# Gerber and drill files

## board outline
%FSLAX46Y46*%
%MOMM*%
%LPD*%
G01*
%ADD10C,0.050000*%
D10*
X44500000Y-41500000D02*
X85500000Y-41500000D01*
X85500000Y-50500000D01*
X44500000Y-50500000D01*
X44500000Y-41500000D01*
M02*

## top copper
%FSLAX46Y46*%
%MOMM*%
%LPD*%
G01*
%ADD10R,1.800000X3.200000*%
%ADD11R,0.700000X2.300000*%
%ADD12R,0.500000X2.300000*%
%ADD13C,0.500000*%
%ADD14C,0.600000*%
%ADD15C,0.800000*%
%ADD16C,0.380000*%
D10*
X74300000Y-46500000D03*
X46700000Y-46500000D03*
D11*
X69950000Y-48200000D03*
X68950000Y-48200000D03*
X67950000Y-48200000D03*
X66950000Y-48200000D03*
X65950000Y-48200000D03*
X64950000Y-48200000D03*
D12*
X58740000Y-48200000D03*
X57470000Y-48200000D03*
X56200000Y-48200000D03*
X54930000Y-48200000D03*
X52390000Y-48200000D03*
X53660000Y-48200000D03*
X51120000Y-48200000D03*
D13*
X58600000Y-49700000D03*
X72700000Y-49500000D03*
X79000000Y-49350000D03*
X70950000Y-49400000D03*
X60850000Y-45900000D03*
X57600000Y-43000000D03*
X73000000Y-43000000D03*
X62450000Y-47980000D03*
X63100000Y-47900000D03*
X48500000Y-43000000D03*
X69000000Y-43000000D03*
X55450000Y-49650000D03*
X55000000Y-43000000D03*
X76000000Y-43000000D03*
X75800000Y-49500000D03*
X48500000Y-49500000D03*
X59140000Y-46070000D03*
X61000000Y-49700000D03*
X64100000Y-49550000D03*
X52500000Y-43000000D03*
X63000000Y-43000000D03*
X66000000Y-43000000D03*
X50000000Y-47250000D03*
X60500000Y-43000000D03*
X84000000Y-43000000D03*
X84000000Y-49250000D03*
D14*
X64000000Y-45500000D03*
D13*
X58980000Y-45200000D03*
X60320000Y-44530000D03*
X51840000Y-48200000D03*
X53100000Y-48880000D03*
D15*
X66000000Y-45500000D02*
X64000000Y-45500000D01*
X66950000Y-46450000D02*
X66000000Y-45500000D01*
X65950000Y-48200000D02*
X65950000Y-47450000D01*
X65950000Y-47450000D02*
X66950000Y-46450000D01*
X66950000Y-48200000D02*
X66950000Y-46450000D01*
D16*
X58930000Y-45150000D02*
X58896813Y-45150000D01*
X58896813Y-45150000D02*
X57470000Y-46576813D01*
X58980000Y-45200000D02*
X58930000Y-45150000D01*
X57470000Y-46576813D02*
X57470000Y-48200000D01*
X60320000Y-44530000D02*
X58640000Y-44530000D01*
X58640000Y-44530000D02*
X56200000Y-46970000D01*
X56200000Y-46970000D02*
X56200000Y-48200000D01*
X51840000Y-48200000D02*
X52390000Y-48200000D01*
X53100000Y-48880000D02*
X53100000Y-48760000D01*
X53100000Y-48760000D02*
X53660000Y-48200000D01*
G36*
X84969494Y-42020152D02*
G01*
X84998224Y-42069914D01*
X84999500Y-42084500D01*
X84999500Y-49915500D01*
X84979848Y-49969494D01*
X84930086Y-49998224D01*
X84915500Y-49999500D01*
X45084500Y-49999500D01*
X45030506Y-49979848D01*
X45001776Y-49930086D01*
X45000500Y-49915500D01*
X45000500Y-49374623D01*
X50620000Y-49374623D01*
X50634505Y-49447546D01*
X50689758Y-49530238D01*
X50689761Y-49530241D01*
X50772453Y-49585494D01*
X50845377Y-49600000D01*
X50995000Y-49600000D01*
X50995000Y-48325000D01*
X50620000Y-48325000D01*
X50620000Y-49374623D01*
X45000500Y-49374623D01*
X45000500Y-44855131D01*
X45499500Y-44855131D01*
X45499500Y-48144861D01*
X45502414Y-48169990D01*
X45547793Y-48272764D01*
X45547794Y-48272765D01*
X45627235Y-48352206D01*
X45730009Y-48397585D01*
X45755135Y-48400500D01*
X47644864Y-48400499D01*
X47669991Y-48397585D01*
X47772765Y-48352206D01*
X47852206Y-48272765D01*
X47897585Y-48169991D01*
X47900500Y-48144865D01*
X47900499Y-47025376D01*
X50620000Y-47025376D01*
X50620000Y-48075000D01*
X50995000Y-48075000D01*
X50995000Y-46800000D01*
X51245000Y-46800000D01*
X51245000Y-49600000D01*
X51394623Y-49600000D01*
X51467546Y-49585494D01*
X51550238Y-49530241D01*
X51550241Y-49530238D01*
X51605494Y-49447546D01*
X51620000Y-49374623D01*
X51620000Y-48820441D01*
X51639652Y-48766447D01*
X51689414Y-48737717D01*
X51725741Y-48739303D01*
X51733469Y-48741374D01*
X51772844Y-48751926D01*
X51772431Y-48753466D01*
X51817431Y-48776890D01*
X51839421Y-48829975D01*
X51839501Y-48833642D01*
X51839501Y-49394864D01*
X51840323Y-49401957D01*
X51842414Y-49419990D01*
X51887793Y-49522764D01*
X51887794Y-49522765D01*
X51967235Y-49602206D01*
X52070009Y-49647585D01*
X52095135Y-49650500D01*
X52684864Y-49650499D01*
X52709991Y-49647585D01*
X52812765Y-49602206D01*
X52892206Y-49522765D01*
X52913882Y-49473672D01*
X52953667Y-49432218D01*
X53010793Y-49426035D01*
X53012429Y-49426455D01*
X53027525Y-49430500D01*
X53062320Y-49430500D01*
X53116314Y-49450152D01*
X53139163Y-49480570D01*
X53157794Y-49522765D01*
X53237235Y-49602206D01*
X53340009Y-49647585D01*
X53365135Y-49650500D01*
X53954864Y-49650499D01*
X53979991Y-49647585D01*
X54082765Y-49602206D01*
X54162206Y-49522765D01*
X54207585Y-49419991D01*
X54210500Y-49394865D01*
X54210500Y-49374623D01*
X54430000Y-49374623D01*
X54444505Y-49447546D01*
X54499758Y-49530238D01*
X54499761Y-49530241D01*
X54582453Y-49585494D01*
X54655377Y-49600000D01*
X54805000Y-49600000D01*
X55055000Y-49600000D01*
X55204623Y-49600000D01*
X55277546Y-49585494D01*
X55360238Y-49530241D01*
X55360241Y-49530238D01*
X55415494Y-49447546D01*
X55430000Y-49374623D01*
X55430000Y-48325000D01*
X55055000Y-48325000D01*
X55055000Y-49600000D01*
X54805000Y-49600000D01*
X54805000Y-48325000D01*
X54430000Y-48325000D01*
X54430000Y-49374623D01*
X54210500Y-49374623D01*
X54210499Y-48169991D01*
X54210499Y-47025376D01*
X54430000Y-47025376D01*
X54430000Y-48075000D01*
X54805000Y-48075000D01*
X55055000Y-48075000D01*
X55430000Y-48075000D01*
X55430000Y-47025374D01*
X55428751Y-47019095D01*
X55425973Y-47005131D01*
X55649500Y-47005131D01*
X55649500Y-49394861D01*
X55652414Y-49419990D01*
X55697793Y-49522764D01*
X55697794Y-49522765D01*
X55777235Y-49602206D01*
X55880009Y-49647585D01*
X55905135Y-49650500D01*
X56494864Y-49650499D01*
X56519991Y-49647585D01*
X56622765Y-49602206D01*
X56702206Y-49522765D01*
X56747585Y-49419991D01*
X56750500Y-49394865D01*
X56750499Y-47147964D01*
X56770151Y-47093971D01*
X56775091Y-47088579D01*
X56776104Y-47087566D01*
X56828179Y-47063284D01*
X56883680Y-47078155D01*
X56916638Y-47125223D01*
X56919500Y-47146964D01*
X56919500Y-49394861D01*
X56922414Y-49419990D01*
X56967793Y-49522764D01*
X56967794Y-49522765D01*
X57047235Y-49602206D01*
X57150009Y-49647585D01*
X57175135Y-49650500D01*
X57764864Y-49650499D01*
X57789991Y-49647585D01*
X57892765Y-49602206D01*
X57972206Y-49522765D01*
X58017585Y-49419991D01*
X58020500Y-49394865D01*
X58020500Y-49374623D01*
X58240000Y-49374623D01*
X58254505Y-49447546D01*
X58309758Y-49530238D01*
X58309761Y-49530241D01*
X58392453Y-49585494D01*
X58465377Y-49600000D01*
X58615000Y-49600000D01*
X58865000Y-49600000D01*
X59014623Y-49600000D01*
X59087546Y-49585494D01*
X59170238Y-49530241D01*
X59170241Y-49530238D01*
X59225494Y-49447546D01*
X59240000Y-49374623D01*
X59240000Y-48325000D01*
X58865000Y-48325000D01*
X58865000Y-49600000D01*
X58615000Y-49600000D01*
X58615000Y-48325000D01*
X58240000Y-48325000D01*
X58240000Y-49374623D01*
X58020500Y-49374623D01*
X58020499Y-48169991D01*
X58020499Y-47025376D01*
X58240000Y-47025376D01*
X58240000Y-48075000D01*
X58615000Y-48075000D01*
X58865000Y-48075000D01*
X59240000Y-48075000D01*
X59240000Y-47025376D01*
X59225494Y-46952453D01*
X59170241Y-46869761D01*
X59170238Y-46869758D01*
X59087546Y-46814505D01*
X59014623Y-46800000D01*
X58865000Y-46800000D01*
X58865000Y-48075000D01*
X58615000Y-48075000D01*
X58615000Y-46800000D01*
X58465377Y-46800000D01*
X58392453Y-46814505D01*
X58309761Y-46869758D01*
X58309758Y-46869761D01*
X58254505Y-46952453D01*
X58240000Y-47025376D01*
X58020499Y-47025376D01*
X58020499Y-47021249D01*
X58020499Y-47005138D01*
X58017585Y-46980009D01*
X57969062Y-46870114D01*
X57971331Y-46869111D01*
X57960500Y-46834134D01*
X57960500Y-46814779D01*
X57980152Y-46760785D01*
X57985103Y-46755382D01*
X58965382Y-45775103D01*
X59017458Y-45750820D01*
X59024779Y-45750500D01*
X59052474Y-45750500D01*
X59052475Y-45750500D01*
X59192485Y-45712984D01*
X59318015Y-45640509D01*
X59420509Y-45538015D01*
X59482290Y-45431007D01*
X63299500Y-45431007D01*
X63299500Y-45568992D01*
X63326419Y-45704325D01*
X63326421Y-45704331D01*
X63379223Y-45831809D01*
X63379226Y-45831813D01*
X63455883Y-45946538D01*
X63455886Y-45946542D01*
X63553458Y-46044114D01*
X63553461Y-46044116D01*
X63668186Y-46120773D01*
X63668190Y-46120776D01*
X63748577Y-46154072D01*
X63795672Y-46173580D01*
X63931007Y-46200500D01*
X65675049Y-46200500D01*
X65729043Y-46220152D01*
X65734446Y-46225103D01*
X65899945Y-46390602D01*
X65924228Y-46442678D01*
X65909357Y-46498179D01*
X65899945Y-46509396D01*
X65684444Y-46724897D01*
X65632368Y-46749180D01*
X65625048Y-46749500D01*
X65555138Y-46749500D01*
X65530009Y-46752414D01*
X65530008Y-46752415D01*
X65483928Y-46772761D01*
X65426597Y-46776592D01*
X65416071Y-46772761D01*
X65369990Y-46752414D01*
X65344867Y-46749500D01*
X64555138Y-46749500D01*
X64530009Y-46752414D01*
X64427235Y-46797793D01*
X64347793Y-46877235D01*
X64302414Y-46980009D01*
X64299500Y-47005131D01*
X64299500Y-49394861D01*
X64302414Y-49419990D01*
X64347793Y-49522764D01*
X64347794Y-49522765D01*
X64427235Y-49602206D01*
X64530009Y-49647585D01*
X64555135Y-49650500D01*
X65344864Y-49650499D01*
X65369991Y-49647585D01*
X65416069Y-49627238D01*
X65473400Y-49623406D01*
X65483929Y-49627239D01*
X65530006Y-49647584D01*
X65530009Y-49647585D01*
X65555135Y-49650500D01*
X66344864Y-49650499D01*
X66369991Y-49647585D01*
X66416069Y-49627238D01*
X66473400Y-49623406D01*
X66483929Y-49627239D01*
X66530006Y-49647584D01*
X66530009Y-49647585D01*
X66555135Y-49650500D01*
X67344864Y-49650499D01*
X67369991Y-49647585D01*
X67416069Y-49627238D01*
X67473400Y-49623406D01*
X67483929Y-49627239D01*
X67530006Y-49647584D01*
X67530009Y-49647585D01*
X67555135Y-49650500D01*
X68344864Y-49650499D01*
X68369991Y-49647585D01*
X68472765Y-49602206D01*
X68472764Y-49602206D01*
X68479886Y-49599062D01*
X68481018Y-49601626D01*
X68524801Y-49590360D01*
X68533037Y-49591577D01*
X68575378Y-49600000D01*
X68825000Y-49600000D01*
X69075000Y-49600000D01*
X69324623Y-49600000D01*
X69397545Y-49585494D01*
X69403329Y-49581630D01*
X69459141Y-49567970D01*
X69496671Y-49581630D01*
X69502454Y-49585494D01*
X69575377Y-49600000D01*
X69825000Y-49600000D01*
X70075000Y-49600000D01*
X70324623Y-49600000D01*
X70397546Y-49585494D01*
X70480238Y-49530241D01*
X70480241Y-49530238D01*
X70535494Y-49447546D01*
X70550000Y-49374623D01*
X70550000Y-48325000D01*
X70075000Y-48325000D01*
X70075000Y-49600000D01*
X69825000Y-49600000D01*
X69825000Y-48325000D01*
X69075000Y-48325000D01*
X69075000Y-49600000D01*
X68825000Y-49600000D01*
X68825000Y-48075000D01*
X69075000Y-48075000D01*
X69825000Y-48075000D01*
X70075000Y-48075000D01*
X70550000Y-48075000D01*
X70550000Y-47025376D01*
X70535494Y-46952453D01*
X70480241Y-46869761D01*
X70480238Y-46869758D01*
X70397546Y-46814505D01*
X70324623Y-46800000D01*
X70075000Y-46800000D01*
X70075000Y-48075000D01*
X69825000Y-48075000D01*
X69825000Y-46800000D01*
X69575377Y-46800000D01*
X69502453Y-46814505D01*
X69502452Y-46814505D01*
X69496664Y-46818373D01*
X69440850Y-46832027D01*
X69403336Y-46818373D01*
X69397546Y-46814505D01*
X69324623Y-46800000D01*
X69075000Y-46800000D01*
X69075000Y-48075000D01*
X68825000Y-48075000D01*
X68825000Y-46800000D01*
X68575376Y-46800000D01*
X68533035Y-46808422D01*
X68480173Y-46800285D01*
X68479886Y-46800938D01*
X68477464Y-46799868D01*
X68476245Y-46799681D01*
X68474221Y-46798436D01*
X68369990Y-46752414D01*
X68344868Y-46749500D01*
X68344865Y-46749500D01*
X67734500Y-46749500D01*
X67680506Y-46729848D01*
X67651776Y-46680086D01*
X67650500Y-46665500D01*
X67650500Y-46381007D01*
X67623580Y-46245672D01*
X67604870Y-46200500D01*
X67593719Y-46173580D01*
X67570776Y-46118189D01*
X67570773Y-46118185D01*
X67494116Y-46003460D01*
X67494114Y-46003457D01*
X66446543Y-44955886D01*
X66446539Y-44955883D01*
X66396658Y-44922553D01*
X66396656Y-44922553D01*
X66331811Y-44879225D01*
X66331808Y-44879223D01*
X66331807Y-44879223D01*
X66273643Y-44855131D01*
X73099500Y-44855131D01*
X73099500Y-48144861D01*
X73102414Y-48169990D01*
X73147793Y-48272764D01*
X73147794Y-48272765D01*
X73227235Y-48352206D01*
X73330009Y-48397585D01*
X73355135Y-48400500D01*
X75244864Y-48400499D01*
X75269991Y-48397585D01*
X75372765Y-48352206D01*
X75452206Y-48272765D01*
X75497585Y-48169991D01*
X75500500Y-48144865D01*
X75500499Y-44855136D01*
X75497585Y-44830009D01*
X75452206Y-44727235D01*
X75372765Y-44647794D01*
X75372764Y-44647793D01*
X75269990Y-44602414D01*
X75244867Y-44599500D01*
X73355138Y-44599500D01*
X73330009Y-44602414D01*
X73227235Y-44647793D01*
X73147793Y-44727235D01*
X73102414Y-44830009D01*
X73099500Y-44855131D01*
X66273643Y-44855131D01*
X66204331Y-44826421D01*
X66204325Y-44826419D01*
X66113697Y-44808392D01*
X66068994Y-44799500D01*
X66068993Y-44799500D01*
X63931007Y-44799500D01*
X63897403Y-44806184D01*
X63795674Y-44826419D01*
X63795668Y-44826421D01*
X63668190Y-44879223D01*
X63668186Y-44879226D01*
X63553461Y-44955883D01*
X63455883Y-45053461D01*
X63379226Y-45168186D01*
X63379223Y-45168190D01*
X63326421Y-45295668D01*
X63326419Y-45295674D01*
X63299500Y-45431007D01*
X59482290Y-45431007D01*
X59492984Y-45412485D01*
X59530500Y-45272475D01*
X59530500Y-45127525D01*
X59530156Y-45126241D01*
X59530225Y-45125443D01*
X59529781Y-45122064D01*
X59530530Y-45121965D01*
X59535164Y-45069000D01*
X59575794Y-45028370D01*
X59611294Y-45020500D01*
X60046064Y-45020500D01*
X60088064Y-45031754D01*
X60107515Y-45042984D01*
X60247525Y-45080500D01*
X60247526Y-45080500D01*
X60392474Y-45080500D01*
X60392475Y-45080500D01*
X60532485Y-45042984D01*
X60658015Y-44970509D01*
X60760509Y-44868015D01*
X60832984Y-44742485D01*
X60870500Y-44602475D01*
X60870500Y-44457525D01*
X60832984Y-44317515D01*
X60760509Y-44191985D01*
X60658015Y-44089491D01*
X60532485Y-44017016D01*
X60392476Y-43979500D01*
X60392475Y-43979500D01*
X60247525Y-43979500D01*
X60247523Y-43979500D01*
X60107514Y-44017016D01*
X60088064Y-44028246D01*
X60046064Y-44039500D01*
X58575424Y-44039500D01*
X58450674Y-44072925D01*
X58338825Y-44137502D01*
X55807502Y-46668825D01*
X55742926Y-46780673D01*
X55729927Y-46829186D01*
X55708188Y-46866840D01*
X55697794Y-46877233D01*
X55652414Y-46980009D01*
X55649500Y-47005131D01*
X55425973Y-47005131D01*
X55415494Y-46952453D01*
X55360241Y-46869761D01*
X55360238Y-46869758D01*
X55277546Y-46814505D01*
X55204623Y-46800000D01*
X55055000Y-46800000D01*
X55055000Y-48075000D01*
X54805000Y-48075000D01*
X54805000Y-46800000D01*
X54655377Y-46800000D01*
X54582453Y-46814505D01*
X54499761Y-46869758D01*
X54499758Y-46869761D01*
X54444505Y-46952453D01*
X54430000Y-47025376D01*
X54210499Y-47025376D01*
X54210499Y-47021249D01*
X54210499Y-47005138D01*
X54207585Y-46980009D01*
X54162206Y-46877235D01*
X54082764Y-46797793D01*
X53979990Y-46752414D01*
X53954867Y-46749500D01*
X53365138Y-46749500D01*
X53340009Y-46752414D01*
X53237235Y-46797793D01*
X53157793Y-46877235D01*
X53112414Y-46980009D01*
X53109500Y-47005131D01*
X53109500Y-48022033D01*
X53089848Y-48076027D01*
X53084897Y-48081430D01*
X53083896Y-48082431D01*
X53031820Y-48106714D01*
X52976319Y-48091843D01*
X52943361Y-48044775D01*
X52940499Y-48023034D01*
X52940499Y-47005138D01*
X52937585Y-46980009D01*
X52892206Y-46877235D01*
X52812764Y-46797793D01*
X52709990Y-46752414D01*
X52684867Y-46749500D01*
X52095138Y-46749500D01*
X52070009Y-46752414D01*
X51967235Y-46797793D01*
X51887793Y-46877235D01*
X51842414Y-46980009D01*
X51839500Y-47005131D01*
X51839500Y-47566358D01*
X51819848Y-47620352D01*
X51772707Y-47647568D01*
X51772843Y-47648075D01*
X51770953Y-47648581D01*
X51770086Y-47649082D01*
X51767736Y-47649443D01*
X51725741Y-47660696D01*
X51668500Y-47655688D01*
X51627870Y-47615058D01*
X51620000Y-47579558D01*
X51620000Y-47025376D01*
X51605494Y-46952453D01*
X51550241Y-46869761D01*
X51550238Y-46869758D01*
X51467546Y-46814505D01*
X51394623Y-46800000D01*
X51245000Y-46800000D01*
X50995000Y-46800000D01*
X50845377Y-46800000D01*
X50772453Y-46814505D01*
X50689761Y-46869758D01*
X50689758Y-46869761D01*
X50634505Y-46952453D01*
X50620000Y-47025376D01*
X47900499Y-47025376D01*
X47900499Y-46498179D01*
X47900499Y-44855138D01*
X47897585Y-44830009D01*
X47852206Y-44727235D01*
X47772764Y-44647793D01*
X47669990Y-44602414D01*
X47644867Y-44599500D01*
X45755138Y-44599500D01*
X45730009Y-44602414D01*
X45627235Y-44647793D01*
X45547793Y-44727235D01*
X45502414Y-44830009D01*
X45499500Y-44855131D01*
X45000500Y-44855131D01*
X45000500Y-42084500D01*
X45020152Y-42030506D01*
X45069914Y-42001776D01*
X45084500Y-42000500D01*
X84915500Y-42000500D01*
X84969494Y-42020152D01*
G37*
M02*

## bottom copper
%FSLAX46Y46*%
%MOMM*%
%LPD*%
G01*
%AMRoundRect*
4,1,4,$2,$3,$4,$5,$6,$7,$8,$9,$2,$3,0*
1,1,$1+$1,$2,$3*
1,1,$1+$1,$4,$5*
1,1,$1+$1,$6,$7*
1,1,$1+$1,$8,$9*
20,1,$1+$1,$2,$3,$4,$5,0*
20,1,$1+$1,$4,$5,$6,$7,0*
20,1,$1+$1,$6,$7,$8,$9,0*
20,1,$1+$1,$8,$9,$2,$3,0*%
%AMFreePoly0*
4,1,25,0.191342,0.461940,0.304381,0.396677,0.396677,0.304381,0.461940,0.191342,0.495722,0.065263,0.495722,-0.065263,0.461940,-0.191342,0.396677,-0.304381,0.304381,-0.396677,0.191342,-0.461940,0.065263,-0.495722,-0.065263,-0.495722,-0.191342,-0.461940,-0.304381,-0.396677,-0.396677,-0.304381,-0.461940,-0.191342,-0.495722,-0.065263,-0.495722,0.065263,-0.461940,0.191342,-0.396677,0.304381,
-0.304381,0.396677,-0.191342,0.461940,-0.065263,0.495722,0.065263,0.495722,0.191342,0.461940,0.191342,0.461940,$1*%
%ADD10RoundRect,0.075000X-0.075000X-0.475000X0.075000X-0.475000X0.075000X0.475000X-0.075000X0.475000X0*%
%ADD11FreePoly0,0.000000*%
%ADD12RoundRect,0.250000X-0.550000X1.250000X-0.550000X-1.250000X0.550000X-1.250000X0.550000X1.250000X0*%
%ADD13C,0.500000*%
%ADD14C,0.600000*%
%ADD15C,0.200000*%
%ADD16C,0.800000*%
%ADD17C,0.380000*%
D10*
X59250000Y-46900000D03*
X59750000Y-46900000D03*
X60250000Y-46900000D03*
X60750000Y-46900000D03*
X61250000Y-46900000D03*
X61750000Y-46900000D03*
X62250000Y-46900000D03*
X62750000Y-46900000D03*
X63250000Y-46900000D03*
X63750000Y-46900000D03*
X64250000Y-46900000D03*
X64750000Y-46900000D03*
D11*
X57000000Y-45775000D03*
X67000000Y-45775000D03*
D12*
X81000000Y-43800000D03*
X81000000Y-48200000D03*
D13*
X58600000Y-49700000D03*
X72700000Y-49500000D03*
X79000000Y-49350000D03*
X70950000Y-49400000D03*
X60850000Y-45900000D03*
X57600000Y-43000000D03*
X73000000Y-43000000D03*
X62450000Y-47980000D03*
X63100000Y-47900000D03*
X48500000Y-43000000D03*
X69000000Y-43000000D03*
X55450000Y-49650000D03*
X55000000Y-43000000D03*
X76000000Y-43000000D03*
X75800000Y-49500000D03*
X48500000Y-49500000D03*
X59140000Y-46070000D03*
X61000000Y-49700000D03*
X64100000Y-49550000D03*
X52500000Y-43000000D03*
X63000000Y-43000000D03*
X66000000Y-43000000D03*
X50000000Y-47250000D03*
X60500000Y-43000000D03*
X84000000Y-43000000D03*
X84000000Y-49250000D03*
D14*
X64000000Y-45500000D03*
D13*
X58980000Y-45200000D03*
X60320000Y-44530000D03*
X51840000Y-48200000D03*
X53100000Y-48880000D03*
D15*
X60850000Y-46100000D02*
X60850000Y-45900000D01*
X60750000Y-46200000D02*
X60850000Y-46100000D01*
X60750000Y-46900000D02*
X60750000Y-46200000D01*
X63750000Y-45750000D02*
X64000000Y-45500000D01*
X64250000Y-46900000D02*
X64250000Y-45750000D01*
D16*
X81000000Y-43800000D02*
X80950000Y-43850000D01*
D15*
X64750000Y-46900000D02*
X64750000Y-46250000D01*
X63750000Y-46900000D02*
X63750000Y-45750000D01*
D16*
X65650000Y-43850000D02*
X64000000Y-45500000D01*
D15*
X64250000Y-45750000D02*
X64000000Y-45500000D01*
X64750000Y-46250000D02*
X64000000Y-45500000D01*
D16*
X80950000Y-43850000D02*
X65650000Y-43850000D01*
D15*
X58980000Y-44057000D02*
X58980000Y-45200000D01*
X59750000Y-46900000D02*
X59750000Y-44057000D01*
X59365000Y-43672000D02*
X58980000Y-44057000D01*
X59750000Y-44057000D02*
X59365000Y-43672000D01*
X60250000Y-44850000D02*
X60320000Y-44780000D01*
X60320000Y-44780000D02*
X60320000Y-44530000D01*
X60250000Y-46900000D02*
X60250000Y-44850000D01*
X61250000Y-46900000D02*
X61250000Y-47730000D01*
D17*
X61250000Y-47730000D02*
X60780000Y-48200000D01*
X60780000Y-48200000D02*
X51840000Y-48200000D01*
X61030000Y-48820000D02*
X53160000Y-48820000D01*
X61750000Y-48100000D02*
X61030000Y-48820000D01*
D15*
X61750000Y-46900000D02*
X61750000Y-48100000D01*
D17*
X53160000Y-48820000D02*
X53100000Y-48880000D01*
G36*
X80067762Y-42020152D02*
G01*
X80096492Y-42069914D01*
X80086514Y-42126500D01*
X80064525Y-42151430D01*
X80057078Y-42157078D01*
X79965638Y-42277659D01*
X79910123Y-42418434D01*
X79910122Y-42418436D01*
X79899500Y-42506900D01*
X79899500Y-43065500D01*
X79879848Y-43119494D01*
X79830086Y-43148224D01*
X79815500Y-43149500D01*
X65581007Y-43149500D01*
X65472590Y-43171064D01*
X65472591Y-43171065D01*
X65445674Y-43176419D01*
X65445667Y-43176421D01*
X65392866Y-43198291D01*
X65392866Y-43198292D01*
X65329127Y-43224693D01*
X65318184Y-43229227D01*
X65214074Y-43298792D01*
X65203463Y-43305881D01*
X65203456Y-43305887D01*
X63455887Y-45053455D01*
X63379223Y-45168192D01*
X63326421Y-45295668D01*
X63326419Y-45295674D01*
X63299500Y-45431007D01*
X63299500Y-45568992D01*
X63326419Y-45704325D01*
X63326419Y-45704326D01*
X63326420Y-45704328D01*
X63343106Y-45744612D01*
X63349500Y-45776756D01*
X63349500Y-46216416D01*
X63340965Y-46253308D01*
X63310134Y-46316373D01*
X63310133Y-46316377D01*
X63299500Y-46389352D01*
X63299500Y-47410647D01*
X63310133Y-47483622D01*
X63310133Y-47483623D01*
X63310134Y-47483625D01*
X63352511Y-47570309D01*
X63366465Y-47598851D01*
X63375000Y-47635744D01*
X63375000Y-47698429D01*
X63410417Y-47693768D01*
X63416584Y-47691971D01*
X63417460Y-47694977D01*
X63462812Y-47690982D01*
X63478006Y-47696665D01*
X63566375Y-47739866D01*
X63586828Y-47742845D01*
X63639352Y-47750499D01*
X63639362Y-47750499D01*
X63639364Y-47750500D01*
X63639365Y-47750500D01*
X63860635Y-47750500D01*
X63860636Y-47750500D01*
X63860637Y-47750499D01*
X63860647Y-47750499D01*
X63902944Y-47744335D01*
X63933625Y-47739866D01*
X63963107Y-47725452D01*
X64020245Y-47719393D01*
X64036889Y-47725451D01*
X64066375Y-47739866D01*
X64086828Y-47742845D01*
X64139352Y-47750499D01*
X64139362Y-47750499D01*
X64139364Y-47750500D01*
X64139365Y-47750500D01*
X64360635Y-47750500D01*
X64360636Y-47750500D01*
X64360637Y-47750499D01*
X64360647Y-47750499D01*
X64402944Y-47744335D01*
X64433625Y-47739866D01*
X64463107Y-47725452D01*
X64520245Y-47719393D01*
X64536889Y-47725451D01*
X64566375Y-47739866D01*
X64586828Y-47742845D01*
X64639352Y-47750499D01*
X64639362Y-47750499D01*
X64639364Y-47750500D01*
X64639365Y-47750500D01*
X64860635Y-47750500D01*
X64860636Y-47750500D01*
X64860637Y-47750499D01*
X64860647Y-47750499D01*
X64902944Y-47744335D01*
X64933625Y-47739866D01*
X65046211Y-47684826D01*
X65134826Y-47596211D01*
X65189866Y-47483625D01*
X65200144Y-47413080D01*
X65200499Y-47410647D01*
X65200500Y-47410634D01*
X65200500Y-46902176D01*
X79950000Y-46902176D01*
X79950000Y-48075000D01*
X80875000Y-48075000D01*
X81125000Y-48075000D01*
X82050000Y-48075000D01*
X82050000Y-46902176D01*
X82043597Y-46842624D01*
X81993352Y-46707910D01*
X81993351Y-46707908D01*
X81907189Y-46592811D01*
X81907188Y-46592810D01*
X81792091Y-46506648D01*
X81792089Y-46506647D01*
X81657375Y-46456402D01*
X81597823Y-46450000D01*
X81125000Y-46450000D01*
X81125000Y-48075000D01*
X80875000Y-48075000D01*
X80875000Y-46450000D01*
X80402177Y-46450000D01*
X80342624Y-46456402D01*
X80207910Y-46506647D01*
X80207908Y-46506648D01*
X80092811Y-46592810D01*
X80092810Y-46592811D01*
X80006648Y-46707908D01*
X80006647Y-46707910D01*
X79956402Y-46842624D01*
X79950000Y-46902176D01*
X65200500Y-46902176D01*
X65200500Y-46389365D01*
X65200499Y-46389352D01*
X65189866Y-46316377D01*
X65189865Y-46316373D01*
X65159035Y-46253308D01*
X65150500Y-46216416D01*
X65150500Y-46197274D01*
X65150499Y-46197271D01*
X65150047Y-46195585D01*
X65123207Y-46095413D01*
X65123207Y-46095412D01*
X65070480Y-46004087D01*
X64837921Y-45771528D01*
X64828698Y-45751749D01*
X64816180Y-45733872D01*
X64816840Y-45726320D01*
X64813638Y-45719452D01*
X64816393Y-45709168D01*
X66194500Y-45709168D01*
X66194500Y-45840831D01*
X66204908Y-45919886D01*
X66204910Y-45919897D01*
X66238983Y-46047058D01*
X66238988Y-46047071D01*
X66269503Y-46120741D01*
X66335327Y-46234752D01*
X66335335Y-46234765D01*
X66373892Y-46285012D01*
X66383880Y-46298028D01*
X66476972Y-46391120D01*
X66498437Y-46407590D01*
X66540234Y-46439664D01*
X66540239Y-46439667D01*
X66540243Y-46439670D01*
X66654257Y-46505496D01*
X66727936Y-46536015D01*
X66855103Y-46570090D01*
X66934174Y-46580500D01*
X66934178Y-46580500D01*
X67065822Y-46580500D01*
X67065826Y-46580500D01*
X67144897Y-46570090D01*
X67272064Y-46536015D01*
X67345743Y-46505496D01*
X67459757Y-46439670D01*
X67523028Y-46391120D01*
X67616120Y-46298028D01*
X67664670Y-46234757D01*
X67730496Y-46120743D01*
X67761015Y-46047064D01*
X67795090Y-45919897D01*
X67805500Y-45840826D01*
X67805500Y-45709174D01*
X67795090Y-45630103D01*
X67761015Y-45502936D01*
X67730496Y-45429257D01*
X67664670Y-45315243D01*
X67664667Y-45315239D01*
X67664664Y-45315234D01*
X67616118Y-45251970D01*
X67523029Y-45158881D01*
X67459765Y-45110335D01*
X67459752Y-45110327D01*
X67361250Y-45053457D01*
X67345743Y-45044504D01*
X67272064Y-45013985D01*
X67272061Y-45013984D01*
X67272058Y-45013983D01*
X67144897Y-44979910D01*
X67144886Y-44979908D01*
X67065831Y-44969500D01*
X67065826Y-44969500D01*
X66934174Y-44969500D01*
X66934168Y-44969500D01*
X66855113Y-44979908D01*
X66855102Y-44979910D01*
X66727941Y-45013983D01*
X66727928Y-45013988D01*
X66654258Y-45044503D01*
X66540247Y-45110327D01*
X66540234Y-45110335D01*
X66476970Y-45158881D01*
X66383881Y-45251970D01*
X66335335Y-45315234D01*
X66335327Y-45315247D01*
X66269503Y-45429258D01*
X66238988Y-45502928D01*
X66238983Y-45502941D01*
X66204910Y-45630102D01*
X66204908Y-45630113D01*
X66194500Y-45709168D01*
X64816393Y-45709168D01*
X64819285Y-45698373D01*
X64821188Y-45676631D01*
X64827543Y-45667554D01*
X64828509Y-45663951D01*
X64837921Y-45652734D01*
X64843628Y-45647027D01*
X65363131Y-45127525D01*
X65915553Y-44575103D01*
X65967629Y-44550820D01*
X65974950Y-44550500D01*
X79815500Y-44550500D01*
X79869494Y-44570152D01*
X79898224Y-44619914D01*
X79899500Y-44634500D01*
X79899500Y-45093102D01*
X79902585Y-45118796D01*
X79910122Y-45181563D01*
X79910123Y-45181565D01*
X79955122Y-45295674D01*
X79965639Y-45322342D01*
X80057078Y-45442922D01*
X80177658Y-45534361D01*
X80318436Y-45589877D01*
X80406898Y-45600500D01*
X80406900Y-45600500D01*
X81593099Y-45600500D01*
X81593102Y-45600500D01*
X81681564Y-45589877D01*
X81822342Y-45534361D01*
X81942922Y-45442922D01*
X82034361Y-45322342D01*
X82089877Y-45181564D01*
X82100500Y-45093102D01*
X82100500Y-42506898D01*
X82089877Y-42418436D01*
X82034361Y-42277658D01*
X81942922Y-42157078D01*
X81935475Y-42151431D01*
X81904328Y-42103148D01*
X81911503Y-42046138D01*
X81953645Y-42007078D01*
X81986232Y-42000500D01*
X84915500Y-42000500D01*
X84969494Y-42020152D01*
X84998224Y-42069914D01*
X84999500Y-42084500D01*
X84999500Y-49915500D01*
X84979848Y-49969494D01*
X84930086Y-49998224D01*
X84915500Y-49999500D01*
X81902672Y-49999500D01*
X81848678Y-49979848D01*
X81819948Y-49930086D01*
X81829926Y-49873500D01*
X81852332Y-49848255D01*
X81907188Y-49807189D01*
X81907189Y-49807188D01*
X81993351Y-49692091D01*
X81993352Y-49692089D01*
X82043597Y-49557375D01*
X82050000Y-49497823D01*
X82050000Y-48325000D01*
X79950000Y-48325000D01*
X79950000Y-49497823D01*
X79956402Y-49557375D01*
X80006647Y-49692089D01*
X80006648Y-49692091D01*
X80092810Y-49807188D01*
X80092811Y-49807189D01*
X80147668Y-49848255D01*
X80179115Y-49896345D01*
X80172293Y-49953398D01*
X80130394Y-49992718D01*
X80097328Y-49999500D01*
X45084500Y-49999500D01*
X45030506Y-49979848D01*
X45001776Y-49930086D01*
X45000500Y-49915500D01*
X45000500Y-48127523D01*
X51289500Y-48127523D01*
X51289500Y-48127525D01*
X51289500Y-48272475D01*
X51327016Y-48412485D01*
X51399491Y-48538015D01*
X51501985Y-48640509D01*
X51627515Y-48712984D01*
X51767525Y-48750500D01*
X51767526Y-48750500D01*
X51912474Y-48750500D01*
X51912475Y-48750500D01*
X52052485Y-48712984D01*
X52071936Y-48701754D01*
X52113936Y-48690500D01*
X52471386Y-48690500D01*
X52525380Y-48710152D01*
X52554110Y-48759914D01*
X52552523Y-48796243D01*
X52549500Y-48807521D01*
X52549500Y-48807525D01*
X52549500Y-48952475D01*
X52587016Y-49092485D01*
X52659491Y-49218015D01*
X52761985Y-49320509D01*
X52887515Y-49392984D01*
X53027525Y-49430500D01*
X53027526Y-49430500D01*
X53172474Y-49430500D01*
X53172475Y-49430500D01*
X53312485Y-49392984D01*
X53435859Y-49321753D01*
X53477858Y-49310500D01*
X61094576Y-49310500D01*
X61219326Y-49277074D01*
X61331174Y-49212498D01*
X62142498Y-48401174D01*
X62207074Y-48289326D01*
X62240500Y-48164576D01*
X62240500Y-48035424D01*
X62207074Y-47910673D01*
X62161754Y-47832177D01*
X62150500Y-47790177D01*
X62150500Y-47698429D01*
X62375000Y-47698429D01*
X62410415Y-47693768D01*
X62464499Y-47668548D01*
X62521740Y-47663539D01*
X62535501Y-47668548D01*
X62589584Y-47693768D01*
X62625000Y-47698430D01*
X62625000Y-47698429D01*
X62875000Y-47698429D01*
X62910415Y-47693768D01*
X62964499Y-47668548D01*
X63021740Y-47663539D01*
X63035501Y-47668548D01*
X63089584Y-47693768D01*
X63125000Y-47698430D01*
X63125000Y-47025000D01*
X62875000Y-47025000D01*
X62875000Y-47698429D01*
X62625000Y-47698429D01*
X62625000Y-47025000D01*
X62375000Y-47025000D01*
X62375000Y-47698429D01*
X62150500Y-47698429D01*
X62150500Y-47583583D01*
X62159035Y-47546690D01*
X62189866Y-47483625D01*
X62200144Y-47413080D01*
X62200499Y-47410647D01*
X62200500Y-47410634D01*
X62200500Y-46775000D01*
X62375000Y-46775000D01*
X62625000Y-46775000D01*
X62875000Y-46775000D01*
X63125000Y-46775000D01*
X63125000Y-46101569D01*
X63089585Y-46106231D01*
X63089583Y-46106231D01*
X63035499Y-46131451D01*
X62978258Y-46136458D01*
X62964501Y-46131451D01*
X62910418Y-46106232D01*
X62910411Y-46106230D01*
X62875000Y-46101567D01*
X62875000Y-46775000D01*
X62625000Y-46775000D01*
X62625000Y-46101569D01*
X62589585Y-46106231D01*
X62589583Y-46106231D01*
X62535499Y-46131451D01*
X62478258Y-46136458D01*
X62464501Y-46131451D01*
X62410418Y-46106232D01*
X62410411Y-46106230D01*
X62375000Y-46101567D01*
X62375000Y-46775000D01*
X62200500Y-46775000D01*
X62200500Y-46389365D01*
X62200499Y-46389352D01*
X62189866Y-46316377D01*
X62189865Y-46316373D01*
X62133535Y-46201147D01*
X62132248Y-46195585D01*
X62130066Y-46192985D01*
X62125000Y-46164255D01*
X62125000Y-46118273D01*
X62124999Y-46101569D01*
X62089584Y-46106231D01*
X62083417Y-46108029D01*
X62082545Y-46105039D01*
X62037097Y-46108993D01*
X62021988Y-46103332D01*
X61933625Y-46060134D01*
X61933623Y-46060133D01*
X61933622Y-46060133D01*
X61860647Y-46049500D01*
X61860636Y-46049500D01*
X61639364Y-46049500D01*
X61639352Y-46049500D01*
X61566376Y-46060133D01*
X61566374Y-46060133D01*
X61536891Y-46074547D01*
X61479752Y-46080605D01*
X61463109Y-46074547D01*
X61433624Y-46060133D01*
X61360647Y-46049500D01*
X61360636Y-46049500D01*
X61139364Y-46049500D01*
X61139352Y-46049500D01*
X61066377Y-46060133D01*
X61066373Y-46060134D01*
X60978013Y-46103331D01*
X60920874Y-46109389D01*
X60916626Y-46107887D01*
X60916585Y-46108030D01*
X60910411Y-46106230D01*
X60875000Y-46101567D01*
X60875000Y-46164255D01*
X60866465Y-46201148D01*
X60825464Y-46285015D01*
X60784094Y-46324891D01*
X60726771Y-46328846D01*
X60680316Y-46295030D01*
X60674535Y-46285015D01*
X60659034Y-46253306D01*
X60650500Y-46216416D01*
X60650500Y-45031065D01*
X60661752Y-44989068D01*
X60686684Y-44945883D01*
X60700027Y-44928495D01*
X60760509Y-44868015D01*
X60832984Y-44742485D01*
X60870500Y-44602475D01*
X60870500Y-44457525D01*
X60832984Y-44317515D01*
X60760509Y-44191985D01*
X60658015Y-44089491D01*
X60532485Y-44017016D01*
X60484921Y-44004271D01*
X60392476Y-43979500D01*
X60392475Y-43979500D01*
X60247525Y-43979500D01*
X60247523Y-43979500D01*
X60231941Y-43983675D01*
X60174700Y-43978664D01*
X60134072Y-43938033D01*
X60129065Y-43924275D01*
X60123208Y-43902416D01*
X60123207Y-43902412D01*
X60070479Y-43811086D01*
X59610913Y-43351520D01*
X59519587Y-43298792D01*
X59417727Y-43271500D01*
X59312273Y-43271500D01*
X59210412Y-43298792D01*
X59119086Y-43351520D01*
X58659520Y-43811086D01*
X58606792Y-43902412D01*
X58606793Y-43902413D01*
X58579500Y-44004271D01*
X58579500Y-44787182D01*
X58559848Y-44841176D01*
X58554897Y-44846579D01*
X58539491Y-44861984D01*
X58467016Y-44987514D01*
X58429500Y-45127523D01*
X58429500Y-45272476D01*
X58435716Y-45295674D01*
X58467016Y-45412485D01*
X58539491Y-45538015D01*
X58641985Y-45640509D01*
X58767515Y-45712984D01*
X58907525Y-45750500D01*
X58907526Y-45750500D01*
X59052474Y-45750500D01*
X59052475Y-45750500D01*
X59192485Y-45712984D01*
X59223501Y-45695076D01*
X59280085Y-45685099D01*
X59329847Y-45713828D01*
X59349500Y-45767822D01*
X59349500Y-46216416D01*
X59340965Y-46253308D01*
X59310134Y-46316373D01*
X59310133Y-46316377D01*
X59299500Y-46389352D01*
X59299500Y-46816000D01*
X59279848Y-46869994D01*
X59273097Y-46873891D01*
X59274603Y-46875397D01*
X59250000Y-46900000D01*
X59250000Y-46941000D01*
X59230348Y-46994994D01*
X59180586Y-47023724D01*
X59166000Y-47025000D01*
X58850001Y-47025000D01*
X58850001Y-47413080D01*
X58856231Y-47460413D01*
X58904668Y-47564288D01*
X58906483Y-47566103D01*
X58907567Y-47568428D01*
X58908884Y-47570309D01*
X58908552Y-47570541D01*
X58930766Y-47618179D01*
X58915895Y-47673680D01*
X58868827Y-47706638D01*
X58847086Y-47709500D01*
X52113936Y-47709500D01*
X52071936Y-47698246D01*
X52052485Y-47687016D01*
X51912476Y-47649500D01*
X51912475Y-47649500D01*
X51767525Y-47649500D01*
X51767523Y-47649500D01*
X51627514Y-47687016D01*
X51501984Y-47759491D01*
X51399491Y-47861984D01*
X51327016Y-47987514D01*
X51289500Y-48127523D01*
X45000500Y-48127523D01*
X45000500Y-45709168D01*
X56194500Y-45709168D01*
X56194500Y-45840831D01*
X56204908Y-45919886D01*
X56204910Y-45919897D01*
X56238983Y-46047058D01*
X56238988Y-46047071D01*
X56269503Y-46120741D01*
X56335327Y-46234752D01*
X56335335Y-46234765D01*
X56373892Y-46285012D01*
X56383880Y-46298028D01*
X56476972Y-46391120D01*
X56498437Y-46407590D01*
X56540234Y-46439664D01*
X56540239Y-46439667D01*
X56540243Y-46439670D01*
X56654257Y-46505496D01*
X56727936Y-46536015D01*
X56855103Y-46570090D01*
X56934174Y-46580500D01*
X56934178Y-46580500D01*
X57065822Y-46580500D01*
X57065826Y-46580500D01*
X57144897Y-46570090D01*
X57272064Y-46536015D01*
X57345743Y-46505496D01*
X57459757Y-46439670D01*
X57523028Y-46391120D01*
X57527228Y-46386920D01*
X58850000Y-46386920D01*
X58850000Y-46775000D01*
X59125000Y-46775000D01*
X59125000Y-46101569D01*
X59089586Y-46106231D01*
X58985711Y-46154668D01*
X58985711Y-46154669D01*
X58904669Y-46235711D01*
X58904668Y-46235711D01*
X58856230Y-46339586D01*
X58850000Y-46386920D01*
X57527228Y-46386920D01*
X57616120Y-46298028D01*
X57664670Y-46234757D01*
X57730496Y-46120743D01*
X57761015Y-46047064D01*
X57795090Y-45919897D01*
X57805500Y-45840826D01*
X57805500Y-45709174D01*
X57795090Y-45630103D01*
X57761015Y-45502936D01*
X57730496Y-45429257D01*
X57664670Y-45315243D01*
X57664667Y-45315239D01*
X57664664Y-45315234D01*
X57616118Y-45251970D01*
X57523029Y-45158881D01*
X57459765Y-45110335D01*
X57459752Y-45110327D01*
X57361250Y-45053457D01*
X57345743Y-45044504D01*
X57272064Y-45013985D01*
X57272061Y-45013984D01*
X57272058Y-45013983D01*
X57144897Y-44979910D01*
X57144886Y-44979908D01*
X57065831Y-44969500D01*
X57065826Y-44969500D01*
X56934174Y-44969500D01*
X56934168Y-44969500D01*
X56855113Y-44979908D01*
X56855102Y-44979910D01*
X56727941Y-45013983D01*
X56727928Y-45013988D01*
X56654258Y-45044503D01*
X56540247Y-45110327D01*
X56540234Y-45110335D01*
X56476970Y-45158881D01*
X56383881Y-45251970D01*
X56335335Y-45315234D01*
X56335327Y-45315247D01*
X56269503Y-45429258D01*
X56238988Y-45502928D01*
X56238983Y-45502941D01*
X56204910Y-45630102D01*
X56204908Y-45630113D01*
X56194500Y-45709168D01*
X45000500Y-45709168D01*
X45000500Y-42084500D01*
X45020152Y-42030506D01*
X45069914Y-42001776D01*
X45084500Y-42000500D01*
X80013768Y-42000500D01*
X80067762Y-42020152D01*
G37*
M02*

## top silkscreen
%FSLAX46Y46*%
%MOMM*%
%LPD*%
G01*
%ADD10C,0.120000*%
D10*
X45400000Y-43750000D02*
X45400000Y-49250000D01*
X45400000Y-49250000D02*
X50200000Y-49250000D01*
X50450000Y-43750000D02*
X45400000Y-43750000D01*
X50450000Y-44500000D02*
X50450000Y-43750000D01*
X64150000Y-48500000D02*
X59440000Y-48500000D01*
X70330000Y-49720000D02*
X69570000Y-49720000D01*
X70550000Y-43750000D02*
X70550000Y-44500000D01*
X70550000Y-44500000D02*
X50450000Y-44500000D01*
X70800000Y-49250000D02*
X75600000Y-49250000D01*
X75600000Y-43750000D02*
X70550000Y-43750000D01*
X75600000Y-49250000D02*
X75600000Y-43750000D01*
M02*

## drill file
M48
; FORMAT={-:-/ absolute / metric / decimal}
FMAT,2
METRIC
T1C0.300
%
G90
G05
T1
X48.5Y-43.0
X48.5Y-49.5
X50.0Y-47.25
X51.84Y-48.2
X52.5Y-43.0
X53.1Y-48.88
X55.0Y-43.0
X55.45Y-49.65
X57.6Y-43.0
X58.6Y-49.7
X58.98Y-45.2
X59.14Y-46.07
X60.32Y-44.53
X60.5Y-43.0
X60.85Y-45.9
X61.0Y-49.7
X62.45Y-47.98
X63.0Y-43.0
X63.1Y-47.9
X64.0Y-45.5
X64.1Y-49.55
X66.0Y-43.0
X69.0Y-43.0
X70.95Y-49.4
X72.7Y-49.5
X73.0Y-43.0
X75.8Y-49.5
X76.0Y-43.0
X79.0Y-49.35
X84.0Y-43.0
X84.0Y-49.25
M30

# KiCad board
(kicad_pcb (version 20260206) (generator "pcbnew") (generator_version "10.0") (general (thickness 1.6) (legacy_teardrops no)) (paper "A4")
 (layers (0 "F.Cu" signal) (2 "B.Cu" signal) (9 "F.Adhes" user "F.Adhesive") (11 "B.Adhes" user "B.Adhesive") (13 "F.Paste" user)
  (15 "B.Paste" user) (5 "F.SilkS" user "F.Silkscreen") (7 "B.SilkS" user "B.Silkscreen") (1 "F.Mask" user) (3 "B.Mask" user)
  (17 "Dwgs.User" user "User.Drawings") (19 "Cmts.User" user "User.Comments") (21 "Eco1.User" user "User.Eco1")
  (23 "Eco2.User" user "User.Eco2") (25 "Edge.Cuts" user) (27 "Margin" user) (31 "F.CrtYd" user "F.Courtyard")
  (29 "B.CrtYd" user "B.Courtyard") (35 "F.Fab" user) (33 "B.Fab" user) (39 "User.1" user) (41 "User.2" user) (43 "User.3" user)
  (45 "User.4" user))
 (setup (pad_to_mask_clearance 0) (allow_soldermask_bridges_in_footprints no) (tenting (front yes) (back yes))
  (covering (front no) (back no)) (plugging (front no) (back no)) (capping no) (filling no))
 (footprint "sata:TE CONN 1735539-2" (layer "F.Cu") (at 60.5 46.5 180)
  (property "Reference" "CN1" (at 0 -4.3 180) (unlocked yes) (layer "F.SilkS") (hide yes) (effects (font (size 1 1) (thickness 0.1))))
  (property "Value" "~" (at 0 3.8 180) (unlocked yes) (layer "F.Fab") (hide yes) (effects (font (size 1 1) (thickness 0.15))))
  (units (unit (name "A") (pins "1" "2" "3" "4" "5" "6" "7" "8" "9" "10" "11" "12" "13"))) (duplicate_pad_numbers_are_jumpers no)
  (fp_line (start 15.1 2.75) (end 15.1 -2.75) (stroke (width 0.12) (type solid)) (layer "F.SilkS"))
  (fp_line (start 15.1 -2.75) (end 10.3 -2.75) (stroke (width 0.12) (type solid)) (layer "F.SilkS"))
  (fp_line (start 10.05 2.75) (end 15.1 2.75) (stroke (width 0.12) (type solid)) (layer "F.SilkS"))
  (fp_line (start 10.05 2) (end 10.05 2.75) (stroke (width 0.12) (type solid)) (layer "F.SilkS"))
  (fp_line (start -3.65 -2) (end 1.06 -2) (stroke (width 0.12) (type solid)) (layer "F.SilkS"))
  (fp_line (start -9.83 -3.22) (end -9.07 -3.22) (stroke (width 0.12) (type solid)) (layer "F.SilkS"))
  (fp_line (start -10.05 2.75) (end -10.05 2) (stroke (width 0.12) (type solid)) (layer "F.SilkS"))
  (fp_line (start -10.05 2) (end 10.05 2) (stroke (width 0.12) (type solid)) (layer "F.SilkS"))
  (fp_line (start -10.3 -2.75) (end -15.1 -2.75) (stroke (width 0.12) (type solid)) (layer "F.SilkS"))
  (fp_line (start -15.1 2.75) (end -10.05 2.75) (stroke (width 0.12) (type solid)) (layer "F.SilkS"))
  (fp_line (start -15.1 -2.75) (end -15.1 2.75) (stroke (width 0.12) (type solid)) (layer "F.SilkS"))
  (pad "" smd rect (at -13.8 0 180) (size 1.8 3.2) (layers "F.Cu" "F.Mask" "F.Paste"))
  (pad "" smd rect (at 13.8 0 180) (size 1.8 3.2) (layers "F.Cu" "F.Mask" "F.Paste"))
  (pad "1" smd rect (at -9.45 -1.7 180) (size 0.7 2.3) (layers "F.Cu" "F.Mask" "F.Paste") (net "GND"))
  (pad "2" smd rect (at -8.45 -1.7 180) (size 0.7 2.3) (layers "F.Cu" "F.Mask" "F.Paste") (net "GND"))
  (pad "3" smd rect (at -7.45 -1.7 180) (size 0.7 2.3) (layers "F.Cu" "F.Mask" "F.Paste") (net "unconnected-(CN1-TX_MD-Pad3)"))
  (pad "4" smd rect (at -6.45 -1.7 180) (size 0.7 2.3) (layers "F.Cu" "F.Mask" "F.Paste") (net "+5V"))
  (pad "5" smd rect (at -5.45 -1.7 180) (size 0.7 2.3) (layers "F.Cu" "F.Mask" "F.Paste") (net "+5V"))
  (pad "6" smd rect (at -4.45 -1.7 180) (size 0.7 2.3) (layers "F.Cu" "F.Mask" "F.Paste") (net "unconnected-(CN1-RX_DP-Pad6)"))
  (pad "7" smd rect (at 1.76 -1.7 180) (size 0.5 2.3) (layers "F.Cu" "F.Mask" "F.Paste") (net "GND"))
  (pad "8" smd rect (at 3.03 -1.7 180) (size 0.5 2.3) (layers "F.Cu" "F.Mask" "F.Paste") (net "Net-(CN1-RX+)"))
  (pad "9" smd rect (at 4.3 -1.7 180) (size 0.5 2.3) (layers "F.Cu" "F.Mask" "F.Paste") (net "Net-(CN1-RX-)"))
  (pad "10" smd rect (at 5.57 -1.7 180) (size 0.5 2.3) (layers "F.Cu" "F.Mask" "F.Paste") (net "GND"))
  (pad "11" smd rect (at 8.11 -1.7 180) (size 0.5 2.3) (layers "F.Cu" "F.Mask" "F.Paste") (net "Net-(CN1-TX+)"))
  (pad "12" smd rect (at 6.84 -1.7 180) (size 0.5 2.3) (layers "F.Cu" "F.Mask" "F.Paste") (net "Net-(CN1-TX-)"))
  (pad "13" smd rect (at 9.38 -1.7 180) (size 0.5 2.3) (layers "F.Cu" "F.Mask" "F.Paste") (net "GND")))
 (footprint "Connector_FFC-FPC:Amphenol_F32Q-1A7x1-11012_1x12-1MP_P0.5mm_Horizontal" (layer "B.Cu") (at 62 44)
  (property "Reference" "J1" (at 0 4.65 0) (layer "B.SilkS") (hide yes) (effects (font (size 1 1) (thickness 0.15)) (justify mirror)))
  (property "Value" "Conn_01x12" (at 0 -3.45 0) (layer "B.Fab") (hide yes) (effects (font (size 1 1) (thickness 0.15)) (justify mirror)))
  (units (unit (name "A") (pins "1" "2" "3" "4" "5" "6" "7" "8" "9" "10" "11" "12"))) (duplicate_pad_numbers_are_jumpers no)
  (pad "1" smd roundrect (at -2.75 2.9) (size 0.3 1.1) (layers "B.Cu" "B.Mask" "B.Paste") (roundrect_rratio 0.25) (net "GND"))
  (pad "2" smd roundrect (at -2.25 2.9) (size 0.3 1.1) (layers "B.Cu" "B.Mask" "B.Paste") (roundrect_rratio 0.25) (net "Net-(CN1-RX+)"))
  (pad "3" smd roundrect (at -1.75 2.9) (size 0.3 1.1) (layers "B.Cu" "B.Mask" "B.Paste") (roundrect_rratio 0.25) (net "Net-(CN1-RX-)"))
  (pad "4" smd roundrect (at -1.25 2.9) (size 0.3 1.1) (layers "B.Cu" "B.Mask" "B.Paste") (roundrect_rratio 0.25) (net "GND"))
  (pad "5" smd roundrect (at -0.75 2.9) (size 0.3 1.1) (layers "B.Cu" "B.Mask" "B.Paste") (roundrect_rratio 0.25) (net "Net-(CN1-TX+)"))
  (pad "6" smd roundrect (at -0.25 2.9) (size 0.3 1.1) (layers "B.Cu" "B.Mask" "B.Paste") (roundrect_rratio 0.25) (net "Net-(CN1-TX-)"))
  (pad "7" smd roundrect (at 0.25 2.9) (size 0.3 1.1) (layers "B.Cu" "B.Mask" "B.Paste") (roundrect_rratio 0.25) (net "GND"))
  (pad "8" smd roundrect (at 0.75 2.9) (size 0.3 1.1) (layers "B.Cu" "B.Mask" "B.Paste") (roundrect_rratio 0.25) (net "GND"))
  (pad "9" smd roundrect (at 1.25 2.9) (size 0.3 1.1) (layers "B.Cu" "B.Mask" "B.Paste") (roundrect_rratio 0.25) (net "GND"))
  (pad "10" smd roundrect (at 1.75 2.9) (size 0.3 1.1) (layers "B.Cu" "B.Mask" "B.Paste") (roundrect_rratio 0.25) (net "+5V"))
  (pad "11" smd roundrect (at 2.25 2.9) (size 0.3 1.1) (layers "B.Cu" "B.Mask" "B.Paste") (roundrect_rratio 0.25) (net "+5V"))
  (pad "12" smd roundrect (at 2.75 2.9) (size 0.3 1.1) (layers "B.Cu" "B.Mask" "B.Paste") (roundrect_rratio 0.25) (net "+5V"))
  (pad "MP" smd custom (at -5 1.775) (size 1 1) (layers "B.Cu" "B.Mask" "B.Paste") (options (clearance outline) (anchor circle))
   (primitives))
  (pad "MP" smd custom (at 5 1.775) (size 1 1) (layers "B.Cu" "B.Mask" "B.Paste") (options (clearance outline) (anchor circle)) (primitives)))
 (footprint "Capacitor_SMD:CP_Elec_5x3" (layer "B.Cu") (at 81 46 -90)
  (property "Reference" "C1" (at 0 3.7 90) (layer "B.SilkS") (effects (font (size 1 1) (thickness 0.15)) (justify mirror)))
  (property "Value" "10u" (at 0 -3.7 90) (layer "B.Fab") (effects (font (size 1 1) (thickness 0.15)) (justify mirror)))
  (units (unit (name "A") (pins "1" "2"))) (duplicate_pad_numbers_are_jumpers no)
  (pad "1" smd roundrect (at -2.2 0 270) (size 3 1.6) (layers "B.Cu" "B.Mask" "B.Paste") (roundrect_rratio 0.15625) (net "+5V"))
  (pad "2" smd roundrect (at 2.2 0 270) (size 3 1.6) (layers "B.Cu" "B.Mask" "B.Paste") (roundrect_rratio 0.15625) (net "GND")))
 (gr_rect (start 44.5 41.5) (end 85.5 50.5) (stroke (width 0.05) (type default)) (fill no) (layer "Edge.Cuts"))
 (via (at 58.6 49.7) (size 0.5) (drill 0.3) (layers "F.Cu" "B.Cu") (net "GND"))
 (via (at 72.7 49.5) (size 0.5) (drill 0.3) (layers "F.Cu" "B.Cu") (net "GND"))
 (via (at 79 49.35) (size 0.5) (drill 0.3) (layers "F.Cu" "B.Cu") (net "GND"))
 (via (at 70.95 49.4) (size 0.5) (drill 0.3) (layers "F.Cu" "B.Cu") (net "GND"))
 (via (at 60.85 45.9) (size 0.5) (drill 0.3) (layers "F.Cu" "B.Cu") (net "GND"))
 (via (at 57.6 43) (size 0.5) (drill 0.3) (layers "F.Cu" "B.Cu") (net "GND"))
 (via (at 73 43) (size 0.5) (drill 0.3) (layers "F.Cu" "B.Cu") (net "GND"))
 (via (at 62.45 47.98) (size 0.5) (drill 0.3) (layers "F.Cu" "B.Cu") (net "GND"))
 (via (at 63.1 47.9) (size 0.5) (drill 0.3) (layers "F.Cu" "B.Cu") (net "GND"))
 (via (at 48.5 43) (size 0.5) (drill 0.3) (layers "F.Cu" "B.Cu") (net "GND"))
 (via (at 69 43) (size 0.5) (drill 0.3) (layers "F.Cu" "B.Cu") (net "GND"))
 (via (at 55.45 49.65) (size 0.5) (drill 0.3) (layers "F.Cu" "B.Cu") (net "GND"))
 (via (at 55 43) (size 0.5) (drill 0.3) (layers "F.Cu" "B.Cu") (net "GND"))
 (via (at 76 43) (size 0.5) (drill 0.3) (layers "F.Cu" "B.Cu") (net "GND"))
 (via (at 75.8 49.5) (size 0.5) (drill 0.3) (layers "F.Cu" "B.Cu") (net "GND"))
 (via (at 48.5 49.5) (size 0.5) (drill 0.3) (layers "F.Cu" "B.Cu") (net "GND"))
 (via (at 59.14 46.07) (size 0.5) (drill 0.3) (layers "F.Cu" "B.Cu") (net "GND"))
 (via (at 61 49.7) (size 0.5) (drill 0.3) (layers "F.Cu" "B.Cu") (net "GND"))
 (via (at 64.1 49.55) (size 0.5) (drill 0.3) (layers "F.Cu" "B.Cu") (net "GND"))
 (via (at 52.5 43) (size 0.5) (drill 0.3) (layers "F.Cu" "B.Cu") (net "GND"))
 (via (at 63 43) (size 0.5) (drill 0.3) (layers "F.Cu" "B.Cu") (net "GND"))
 (via (at 66 43) (size 0.5) (drill 0.3) (layers "F.Cu" "B.Cu") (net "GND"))
 (via (at 50 47.25) (size 0.5) (drill 0.3) (layers "F.Cu" "B.Cu") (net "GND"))
 (via (at 60.5 43) (size 0.5) (drill 0.3) (layers "F.Cu" "B.Cu") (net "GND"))
 (via (at 84 43) (size 0.5) (drill 0.3) (layers "F.Cu" "B.Cu") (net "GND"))
 (via (at 84 49.25) (size 0.5) (drill 0.3) (layers "F.Cu" "B.Cu") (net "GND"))
 (segment (start 60.85 46.1) (end 60.85 45.9) (width 0.2) (layer "B.Cu") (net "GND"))
 (segment (start 60.75 46.2) (end 60.85 46.1) (width 0.2) (layer "B.Cu") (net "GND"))
 (segment (start 60.75 46.9) (end 60.75 46.2) (width 0.2) (layer "B.Cu") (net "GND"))
 (segment (start 66 45.5) (end 64 45.5) (width 0.8) (layer "F.Cu") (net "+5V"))
 (segment (start 66.95 46.45) (end 66 45.5) (width 0.8) (layer "F.Cu") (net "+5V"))
 (segment (start 65.95 48.2) (end 65.95 47.45) (width 0.8) (layer "F.Cu") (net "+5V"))
 (segment (start 65.95 47.45) (end 66.95 46.45) (width 0.8) (layer "F.Cu") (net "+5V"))
 (segment (start 66.95 48.2) (end 66.95 46.45) (width 0.8) (layer "F.Cu") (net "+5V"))
 (via (at 64 45.5) (size 0.6) (drill 0.3) (layers "F.Cu" "B.Cu") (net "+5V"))
 (segment (start 63.75 45.75) (end 64 45.5) (width 0.2) (layer "B.Cu") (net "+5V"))
 (segment (start 64.25 46.9) (end 64.25 45.75) (width 0.2) (layer "B.Cu") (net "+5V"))
 (segment (start 81 43.8) (end 80.95 43.85) (width 0.8) (layer "B.Cu") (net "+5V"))
 (segment (start 64.75 46.9) (end 64.75 46.25) (width 0.2) (layer "B.Cu") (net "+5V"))
 (segment (start 63.75 46.9) (end 63.75 45.75) (width 0.2) (layer "B.Cu") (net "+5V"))
 (segment (start 65.65 43.85) (end 64 45.5) (width 0.8) (layer "B.Cu") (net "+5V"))
 (segment (start 64.25 45.75) (end 64 45.5) (width 0.2) (layer "B.Cu") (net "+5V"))
 (segment (start 64.75 46.25) (end 64 45.5) (width 0.2) (layer "B.Cu") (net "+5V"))
 (segment (start 80.95 43.85) (end 65.65 43.85) (width 0.8) (layer "B.Cu") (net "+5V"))
 (segment (start 58.93 45.15) (end 58.896813 45.15) (width 0.38) (layer "F.Cu") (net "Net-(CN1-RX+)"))
 (segment (start 58.896813 45.15) (end 57.47 46.576813) (width 0.38) (layer "F.Cu") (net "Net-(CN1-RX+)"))
 (segment (start 58.98 45.2) (end 58.93 45.15) (width 0.38) (layer "F.Cu") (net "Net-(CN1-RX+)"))
 (segment (start 57.47 46.576813) (end 57.47 48.2) (width 0.38) (layer "F.Cu") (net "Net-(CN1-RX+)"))
 (via (at 58.98 45.2) (size 0.5) (drill 0.3) (layers "F.Cu" "B.Cu") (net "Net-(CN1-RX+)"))
 (segment (start 58.98 44.057) (end 58.98 45.2) (width 0.2) (layer "B.Cu") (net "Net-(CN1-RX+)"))
 (segment (start 59.75 46.9) (end 59.75 44.057) (width 0.2) (layer "B.Cu") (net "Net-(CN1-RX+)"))
 (segment (start 59.365 43.672) (end 58.98 44.057) (width 0.2) (layer "B.Cu") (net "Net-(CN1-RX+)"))
 (segment (start 59.75 44.057) (end 59.365 43.672) (width 0.2) (layer "B.Cu") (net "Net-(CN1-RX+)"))
 (segment (start 60.32 44.53) (end 58.64 44.53) (width 0.38) (layer "F.Cu") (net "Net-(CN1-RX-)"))
 (segment (start 58.64 44.53) (end 56.2 46.97) (width 0.38) (layer "F.Cu") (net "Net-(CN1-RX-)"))
 (segment (start 56.2 46.97) (end 56.2 48.2) (width 0.38) (layer "F.Cu") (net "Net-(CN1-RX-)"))
 (via (at 60.32 44.53) (size 0.5) (drill 0.3) (layers "F.Cu" "B.Cu") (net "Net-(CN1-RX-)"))
 (segment (start 60.25 44.85) (end 60.32 44.78) (width 0.2) (layer "B.Cu") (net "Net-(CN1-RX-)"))
 (segment (start 60.32 44.78) (end 60.32 44.53) (width 0.2) (layer "B.Cu") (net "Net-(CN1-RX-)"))
 (segment (start 60.25 46.9) (end 60.25 44.85) (width 0.2) (layer "B.Cu") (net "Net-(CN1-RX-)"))
 (segment (start 51.84 48.2) (end 52.39 48.2) (width 0.38) (layer "F.Cu") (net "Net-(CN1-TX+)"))
 (via (at 51.84 48.2) (size 0.5) (drill 0.3) (layers "F.Cu" "B.Cu") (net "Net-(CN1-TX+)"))
 (segment (start 61.25 46.9) (end 61.25 47.73) (width 0.2) (layer "B.Cu") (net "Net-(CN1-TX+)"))
 (segment (start 61.25 47.73) (end 60.78 48.2) (width 0.38) (layer "B.Cu") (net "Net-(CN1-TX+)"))
 (segment (start 60.78 48.2) (end 51.84 48.2) (width 0.38) (layer "B.Cu") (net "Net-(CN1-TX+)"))
 (segment (start 53.1 48.88) (end 53.1 48.76) (width 0.38) (layer "F.Cu") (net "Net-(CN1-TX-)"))
 (segment (start 53.1 48.76) (end 53.66 48.2) (width 0.38) (layer "F.Cu") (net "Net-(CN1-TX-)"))
 (via (at 53.1 48.88) (size 0.5) (drill 0.3) (layers "F.Cu" "B.Cu") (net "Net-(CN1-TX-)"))
 (segment (start 61.03 48.82) (end 53.16 48.82) (width 0.38) (layer "B.Cu") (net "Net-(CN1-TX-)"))
 (segment (start 61.75 48.1) (end 61.03 48.82) (width 0.38) (layer "B.Cu") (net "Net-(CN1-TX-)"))
 (segment (start 61.75 46.9) (end 61.75 48.1) (width 0.2) (layer "B.Cu") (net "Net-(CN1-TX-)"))
 (segment (start 53.16 48.82) (end 53.1 48.88) (width 0.38) (layer "B.Cu") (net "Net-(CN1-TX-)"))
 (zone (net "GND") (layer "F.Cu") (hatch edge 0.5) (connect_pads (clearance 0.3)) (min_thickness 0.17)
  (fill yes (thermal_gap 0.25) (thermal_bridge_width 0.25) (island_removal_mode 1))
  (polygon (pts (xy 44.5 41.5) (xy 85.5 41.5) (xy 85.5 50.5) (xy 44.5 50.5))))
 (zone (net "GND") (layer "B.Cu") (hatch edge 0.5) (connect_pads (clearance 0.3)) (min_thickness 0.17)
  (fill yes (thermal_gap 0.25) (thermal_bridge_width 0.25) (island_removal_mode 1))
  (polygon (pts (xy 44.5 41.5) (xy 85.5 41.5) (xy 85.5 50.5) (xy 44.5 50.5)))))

